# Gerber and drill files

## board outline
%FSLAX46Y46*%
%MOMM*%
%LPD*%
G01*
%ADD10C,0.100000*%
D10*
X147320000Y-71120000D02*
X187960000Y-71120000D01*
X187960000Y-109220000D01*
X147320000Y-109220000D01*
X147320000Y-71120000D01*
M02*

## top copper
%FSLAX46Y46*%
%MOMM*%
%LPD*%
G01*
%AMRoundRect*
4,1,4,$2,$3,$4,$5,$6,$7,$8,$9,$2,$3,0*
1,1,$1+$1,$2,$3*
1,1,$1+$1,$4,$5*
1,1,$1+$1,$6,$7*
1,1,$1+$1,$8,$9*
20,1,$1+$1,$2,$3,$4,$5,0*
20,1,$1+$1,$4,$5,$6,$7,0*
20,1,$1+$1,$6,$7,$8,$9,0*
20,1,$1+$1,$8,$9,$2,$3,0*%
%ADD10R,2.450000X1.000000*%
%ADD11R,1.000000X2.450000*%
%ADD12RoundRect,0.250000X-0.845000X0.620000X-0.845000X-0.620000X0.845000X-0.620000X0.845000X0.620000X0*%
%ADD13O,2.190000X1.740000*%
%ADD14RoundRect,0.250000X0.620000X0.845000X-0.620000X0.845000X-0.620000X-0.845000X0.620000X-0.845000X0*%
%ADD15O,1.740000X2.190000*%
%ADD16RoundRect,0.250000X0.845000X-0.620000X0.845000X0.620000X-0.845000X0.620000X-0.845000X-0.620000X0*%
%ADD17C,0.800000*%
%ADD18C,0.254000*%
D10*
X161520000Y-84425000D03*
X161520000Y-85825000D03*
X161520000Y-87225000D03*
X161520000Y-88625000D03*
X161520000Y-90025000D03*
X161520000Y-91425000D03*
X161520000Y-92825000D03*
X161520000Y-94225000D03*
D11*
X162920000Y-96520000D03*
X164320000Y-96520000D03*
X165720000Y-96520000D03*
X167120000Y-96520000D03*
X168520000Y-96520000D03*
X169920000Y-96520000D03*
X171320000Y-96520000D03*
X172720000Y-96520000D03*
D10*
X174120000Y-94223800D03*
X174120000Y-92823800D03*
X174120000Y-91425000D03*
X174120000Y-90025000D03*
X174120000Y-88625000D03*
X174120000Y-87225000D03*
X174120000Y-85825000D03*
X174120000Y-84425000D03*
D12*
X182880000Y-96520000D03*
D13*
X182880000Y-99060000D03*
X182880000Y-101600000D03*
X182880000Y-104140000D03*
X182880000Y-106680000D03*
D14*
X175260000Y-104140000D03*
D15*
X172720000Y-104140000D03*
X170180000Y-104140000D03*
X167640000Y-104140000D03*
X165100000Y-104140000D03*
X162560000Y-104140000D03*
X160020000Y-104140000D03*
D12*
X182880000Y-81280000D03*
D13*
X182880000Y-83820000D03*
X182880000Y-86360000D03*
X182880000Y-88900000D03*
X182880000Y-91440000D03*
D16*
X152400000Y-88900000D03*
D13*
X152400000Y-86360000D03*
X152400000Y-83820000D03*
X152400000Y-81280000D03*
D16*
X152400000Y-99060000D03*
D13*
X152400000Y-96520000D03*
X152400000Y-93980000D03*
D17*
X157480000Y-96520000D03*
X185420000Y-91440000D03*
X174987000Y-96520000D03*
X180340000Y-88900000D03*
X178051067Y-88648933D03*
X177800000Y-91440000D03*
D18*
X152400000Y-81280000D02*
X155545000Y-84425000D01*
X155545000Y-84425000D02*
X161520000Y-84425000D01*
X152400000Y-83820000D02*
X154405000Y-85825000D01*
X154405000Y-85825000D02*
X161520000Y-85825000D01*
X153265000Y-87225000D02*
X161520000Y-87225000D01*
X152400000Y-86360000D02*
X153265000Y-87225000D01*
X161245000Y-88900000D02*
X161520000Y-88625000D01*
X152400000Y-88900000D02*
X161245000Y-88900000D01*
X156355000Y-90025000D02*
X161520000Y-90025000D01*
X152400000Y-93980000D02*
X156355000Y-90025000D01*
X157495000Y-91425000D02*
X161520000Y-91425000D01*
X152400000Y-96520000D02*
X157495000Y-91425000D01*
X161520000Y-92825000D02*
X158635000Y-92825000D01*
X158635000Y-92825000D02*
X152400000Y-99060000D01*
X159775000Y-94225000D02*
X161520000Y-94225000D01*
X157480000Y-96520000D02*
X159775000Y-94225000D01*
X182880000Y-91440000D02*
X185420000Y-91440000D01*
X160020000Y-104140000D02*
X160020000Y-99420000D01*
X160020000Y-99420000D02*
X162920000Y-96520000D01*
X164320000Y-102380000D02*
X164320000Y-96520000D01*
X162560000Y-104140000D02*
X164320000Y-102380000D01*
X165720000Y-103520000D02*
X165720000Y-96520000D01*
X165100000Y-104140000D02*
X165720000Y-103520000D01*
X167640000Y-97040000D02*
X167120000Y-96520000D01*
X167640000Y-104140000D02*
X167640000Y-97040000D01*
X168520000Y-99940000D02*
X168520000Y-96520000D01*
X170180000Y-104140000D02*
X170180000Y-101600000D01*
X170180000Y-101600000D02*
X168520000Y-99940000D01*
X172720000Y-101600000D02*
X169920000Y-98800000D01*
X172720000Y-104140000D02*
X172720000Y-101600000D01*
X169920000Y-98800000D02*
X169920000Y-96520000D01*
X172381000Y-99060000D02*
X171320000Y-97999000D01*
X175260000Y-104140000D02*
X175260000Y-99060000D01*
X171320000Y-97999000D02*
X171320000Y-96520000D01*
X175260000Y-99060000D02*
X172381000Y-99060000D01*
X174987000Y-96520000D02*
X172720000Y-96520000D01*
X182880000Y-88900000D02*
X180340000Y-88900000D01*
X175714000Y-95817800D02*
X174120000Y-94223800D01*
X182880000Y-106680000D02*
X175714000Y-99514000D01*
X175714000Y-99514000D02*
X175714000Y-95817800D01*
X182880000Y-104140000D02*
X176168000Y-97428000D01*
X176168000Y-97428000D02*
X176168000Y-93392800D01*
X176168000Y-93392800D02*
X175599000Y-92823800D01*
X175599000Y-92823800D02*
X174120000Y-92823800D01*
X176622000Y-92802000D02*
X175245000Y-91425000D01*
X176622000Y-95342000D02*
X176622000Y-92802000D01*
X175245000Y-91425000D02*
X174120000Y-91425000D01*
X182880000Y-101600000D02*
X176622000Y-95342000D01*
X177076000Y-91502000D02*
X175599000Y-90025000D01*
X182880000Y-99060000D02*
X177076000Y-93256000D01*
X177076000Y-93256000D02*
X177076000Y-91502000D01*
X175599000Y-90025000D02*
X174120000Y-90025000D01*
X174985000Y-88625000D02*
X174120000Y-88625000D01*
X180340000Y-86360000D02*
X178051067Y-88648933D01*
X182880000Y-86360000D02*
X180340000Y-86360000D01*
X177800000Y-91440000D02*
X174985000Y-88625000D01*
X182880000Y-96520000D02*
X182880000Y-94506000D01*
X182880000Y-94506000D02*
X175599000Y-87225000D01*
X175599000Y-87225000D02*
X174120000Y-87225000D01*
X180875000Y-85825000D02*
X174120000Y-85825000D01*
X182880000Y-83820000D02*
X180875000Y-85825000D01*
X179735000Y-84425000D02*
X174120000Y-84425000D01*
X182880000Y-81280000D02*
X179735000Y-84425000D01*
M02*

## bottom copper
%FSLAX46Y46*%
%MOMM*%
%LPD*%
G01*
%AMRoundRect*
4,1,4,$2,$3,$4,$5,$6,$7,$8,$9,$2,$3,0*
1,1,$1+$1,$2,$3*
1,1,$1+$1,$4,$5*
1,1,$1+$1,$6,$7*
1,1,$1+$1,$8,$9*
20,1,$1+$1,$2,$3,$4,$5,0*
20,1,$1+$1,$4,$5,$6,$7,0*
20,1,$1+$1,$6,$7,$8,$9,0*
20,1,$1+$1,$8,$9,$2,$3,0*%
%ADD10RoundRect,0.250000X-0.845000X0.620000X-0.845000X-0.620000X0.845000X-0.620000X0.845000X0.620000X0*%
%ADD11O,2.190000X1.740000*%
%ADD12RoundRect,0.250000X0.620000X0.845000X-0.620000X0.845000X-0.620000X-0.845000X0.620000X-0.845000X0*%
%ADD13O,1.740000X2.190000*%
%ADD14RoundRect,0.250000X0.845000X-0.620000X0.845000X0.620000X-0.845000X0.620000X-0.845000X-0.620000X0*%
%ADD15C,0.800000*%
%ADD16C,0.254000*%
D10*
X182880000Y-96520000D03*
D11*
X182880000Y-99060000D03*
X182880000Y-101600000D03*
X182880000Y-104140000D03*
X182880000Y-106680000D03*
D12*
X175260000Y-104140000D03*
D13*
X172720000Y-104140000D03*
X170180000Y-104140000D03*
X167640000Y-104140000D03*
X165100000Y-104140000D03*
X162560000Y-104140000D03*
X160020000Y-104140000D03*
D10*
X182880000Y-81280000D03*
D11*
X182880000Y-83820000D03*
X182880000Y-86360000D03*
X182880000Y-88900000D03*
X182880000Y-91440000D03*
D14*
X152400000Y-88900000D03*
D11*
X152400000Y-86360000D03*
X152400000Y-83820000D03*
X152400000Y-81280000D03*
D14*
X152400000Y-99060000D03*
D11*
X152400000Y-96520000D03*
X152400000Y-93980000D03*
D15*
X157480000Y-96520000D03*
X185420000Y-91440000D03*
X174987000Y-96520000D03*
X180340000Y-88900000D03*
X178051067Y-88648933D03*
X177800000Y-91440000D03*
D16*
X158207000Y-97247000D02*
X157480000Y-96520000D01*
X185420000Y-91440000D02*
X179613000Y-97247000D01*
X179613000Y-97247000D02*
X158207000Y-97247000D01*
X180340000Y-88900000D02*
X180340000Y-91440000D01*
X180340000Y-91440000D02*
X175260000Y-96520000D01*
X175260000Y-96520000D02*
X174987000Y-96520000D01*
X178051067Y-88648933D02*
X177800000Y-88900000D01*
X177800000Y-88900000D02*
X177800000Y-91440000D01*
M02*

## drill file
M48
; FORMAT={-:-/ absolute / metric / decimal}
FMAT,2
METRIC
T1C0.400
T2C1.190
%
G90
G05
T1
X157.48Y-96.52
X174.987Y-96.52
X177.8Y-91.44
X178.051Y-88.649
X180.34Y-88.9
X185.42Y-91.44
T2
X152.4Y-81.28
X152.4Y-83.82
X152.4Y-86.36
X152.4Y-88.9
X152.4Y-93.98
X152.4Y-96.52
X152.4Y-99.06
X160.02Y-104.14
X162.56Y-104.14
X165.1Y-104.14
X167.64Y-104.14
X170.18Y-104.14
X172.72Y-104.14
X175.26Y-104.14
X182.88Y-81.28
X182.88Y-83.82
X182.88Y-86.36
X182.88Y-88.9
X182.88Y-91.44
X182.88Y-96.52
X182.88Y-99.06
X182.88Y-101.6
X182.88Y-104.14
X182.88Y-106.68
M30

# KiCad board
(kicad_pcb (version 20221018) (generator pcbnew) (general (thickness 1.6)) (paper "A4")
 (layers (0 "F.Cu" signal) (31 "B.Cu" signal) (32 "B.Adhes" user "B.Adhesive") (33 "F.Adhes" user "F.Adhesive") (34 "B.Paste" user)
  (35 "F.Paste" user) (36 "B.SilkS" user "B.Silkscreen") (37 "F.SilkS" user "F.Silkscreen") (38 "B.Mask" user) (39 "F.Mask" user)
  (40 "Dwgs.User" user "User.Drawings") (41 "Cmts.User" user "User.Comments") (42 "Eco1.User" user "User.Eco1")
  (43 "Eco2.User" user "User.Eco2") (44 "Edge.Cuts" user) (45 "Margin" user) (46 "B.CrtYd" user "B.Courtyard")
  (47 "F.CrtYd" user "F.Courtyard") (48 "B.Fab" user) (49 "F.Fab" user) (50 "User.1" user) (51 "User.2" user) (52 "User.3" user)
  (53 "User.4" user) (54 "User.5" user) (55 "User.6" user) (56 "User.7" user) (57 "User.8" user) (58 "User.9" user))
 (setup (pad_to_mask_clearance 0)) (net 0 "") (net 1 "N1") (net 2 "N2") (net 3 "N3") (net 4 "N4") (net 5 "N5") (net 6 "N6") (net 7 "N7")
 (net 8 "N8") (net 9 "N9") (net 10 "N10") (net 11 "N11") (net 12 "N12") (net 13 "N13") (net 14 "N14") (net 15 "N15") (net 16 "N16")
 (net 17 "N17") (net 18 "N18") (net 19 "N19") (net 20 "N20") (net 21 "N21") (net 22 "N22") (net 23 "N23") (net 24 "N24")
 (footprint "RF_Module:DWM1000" (layer "F.Cu") (at 167.82 85.2238)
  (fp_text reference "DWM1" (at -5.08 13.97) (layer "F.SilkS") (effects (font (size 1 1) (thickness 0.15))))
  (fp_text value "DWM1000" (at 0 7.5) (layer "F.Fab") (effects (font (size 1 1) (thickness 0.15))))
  (pad "1" smd rect (at -6.3 -0.7988 90) (size 1 2.45) (layers "F.Cu" "F.Paste" "F.Mask") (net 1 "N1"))
  (pad "2" smd rect (at -6.3 0.6012 90) (size 1 2.45) (layers "F.Cu" "F.Paste" "F.Mask") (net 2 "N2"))
  (pad "3" smd rect (at -6.3 2.0012 90) (size 1 2.45) (layers "F.Cu" "F.Paste" "F.Mask") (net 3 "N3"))
  (pad "4" smd rect (at -6.3 3.4012 90) (size 1 2.45) (layers "F.Cu" "F.Paste" "F.Mask") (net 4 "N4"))
  (pad "5" smd rect (at -6.3 4.8012 90) (size 1 2.45) (layers "F.Cu" "F.Paste" "F.Mask") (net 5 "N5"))
  (pad "6" smd rect (at -6.3 6.2012 90) (size 1 2.45) (layers "F.Cu" "F.Paste" "F.Mask") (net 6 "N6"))
  (pad "7" smd rect (at -6.3 7.6012 90) (size 1 2.45) (layers "F.Cu" "F.Paste" "F.Mask") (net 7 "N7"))
  (pad "8" smd rect (at -6.3 9.0012 90) (size 1 2.45) (layers "F.Cu" "F.Paste" "F.Mask") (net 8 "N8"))
  (pad "9" smd rect (at -4.9 11.2962) (size 1 2.45) (layers "F.Cu" "F.Paste" "F.Mask") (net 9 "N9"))
  (pad "10" smd rect (at -3.5 11.2962) (size 1 2.45) (layers "F.Cu" "F.Paste" "F.Mask") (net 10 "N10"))
  (pad "11" smd rect (at -2.1 11.2962) (size 1 2.45) (layers "F.Cu" "F.Paste" "F.Mask") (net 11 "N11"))
  (pad "12" smd rect (at -0.7 11.2962) (size 1 2.45) (layers "F.Cu" "F.Paste" "F.Mask") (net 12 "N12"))
  (pad "13" smd rect (at 0.7 11.2962) (size 1 2.45) (layers "F.Cu" "F.Paste" "F.Mask") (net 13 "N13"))
  (pad "14" smd rect (at 2.1 11.2962) (size 1 2.45) (layers "F.Cu" "F.Paste" "F.Mask") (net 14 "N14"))
  (pad "15" smd rect (at 3.5 11.2962) (size 1 2.45) (layers "F.Cu" "F.Paste" "F.Mask") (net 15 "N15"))
  (pad "16" smd rect (at 4.9 11.2962) (size 1 2.45) (layers "F.Cu" "F.Paste" "F.Mask") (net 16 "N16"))
  (pad "17" smd rect (at 6.3 9 90) (size 1 2.45) (layers "F.Cu" "F.Paste" "F.Mask") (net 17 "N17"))
  (pad "18" smd rect (at 6.3 7.6 90) (size 1 2.45) (layers "F.Cu" "F.Paste" "F.Mask") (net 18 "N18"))
  (pad "19" smd rect (at 6.3 6.2012 90) (size 1 2.45) (layers "F.Cu" "F.Paste" "F.Mask") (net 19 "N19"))
  (pad "20" smd rect (at 6.3 4.8012 90) (size 1 2.45) (layers "F.Cu" "F.Paste" "F.Mask") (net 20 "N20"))
  (pad "21" smd rect (at 6.3 3.4012 90) (size 1 2.45) (layers "F.Cu" "F.Paste" "F.Mask") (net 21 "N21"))
  (pad "22" smd rect (at 6.3 2.0012 90) (size 1 2.45) (layers "F.Cu" "F.Paste" "F.Mask") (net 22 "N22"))
  (pad "23" smd rect (at 6.3 0.6012 90) (size 1 2.45) (layers "F.Cu" "F.Paste" "F.Mask") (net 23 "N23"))
  (pad "24" smd rect (at 6.3 -0.7988 90) (size 1 2.45) (layers "F.Cu" "F.Paste" "F.Mask") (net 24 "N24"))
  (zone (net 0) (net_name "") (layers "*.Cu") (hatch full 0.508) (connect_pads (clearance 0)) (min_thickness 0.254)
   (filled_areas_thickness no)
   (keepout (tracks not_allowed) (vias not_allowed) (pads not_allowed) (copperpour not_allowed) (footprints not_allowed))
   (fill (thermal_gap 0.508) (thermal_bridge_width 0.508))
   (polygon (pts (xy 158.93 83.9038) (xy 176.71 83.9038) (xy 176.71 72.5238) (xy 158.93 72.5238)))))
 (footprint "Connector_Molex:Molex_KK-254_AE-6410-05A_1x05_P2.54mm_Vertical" (layer "F.Cu") (at 182.88 96.52 -90)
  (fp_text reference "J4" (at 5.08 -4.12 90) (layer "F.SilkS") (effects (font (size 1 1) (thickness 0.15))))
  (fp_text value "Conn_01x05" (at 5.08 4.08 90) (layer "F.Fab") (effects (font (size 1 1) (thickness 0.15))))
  (pad "1" thru_hole roundrect (at 0 0 270) (size 1.74 2.19) (drill 1.19) (layers "*.Cu" "*.Mask") (roundrect_rratio 0.1436781609)
   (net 22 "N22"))
  (pad "2" thru_hole oval (at 2.54 0 270) (size 1.74 2.19) (drill 1.19) (layers "*.Cu" "*.Mask") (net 20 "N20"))
  (pad "3" thru_hole oval (at 5.08 0 270) (size 1.74 2.19) (drill 1.19) (layers "*.Cu" "*.Mask") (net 19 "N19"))
  (pad "4" thru_hole oval (at 7.62 0 270) (size 1.74 2.19) (drill 1.19) (layers "*.Cu" "*.Mask") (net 18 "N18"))
  (pad "5" thru_hole oval (at 10.16 0 270) (size 1.74 2.19) (drill 1.19) (layers "*.Cu" "*.Mask") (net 17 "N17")))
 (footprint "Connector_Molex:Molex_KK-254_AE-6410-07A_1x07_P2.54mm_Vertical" (layer "F.Cu") (at 175.26 104.14 180)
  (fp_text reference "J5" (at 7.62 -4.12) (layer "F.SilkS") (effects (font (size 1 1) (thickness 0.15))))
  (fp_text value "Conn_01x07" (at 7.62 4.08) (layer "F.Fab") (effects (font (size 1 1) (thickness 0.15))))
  (pad "1" thru_hole roundrect (at 0 0 180) (size 1.74 2.19) (drill 1.19) (layers "*.Cu" "*.Mask") (roundrect_rratio 0.1436781609)
   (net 15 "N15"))
  (pad "2" thru_hole oval (at 2.54 0 180) (size 1.74 2.19) (drill 1.19) (layers "*.Cu" "*.Mask") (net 14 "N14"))
  (pad "3" thru_hole oval (at 5.08 0 180) (size 1.74 2.19) (drill 1.19) (layers "*.Cu" "*.Mask") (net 13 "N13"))
  (pad "4" thru_hole oval (at 7.62 0 180) (size 1.74 2.19) (drill 1.19) (layers "*.Cu" "*.Mask") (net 12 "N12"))
  (pad "5" thru_hole oval (at 10.16 0 180) (size 1.74 2.19) (drill 1.19) (layers "*.Cu" "*.Mask") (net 11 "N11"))
  (pad "6" thru_hole oval (at 12.7 0 180) (size 1.74 2.19) (drill 1.19) (layers "*.Cu" "*.Mask") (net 10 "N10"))
  (pad "7" thru_hole oval (at 15.24 0 180) (size 1.74 2.19) (drill 1.19) (layers "*.Cu" "*.Mask") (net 9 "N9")))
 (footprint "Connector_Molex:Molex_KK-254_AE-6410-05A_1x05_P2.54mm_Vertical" (layer "F.Cu") (at 182.88 81.28 -90)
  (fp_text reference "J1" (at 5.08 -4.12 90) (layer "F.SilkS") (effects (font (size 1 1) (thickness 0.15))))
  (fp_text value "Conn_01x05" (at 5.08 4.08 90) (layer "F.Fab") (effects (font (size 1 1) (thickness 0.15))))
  (pad "1" thru_hole roundrect (at 0 0 270) (size 1.74 2.19) (drill 1.19) (layers "*.Cu" "*.Mask") (roundrect_rratio 0.1436781609)
   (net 24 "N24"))
  (pad "2" thru_hole oval (at 2.54 0 270) (size 1.74 2.19) (drill 1.19) (layers "*.Cu" "*.Mask") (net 23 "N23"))
  (pad "3" thru_hole oval (at 5.08 0 270) (size 1.74 2.19) (drill 1.19) (layers "*.Cu" "*.Mask") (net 21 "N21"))
  (pad "4" thru_hole oval (at 7.62 0 270) (size 1.74 2.19) (drill 1.19) (layers "*.Cu" "*.Mask") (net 16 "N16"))
  (pad "5" thru_hole oval (at 10.16 0 270) (size 1.74 2.19) (drill 1.19) (layers "*.Cu" "*.Mask") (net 8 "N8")))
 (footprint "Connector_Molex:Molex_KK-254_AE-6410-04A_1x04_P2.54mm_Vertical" (layer "F.Cu") (at 152.4 88.9 90)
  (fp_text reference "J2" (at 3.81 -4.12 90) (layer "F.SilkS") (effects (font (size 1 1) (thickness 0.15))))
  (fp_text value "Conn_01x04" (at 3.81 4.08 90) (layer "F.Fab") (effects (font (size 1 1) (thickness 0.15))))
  (pad "1" thru_hole roundrect (at 0 0 90) (size 1.74 2.19) (drill 1.19) (layers "*.Cu" "*.Mask") (roundrect_rratio 0.1436781609)
   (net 4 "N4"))
  (pad "2" thru_hole oval (at 2.54 0 90) (size 1.74 2.19) (drill 1.19) (layers "*.Cu" "*.Mask") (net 3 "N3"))
  (pad "3" thru_hole oval (at 5.08 0 90) (size 1.74 2.19) (drill 1.19) (layers "*.Cu" "*.Mask") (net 2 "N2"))
  (pad "4" thru_hole oval (at 7.62 0 90) (size 1.74 2.19) (drill 1.19) (layers "*.Cu" "*.Mask") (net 1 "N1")))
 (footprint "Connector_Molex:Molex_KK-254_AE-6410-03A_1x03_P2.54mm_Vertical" (layer "F.Cu") (at 152.4 99.06 90)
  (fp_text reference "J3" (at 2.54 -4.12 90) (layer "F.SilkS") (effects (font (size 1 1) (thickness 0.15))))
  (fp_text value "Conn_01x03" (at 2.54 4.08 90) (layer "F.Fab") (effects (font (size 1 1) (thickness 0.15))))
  (pad "1" thru_hole roundrect (at 0 0 90) (size 1.74 2.19) (drill 1.19) (layers "*.Cu" "*.Mask") (roundrect_rratio 0.1436781609)
   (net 7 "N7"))
  (pad "2" thru_hole oval (at 2.54 0 90) (size 1.74 2.19) (drill 1.19) (layers "*.Cu" "*.Mask") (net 6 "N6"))
  (pad "3" thru_hole oval (at 5.08 0 90) (size 1.74 2.19) (drill 1.19) (layers "*.Cu" "*.Mask") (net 5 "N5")))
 (gr_rect (start 147.32 71.12) (end 187.96 109.22) (stroke (width 0.1) (type default)) (fill none) (layer "Edge.Cuts"))
 (segment (start 152.4 81.28) (end 155.545 84.425) (width 0.254) (layer "F.Cu") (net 1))
 (segment (start 155.545 84.425) (end 161.52 84.425) (width 0.254) (layer "F.Cu") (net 1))
 (segment (start 152.4 83.82) (end 154.405 85.825) (width 0.254) (layer "F.Cu") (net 2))
 (segment (start 154.405 85.825) (end 161.52 85.825) (width 0.254) (layer "F.Cu") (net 2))
 (segment (start 153.265 87.225) (end 161.52 87.225) (width 0.254) (layer "F.Cu") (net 3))
 (segment (start 152.4 86.36) (end 153.265 87.225) (width 0.254) (layer "F.Cu") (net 3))
 (segment (start 161.245 88.9) (end 161.52 88.625) (width 0.254) (layer "F.Cu") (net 4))
 (segment (start 152.4 88.9) (end 161.245 88.9) (width 0.254) (layer "F.Cu") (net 4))
 (segment (start 156.355 90.025) (end 161.52 90.025) (width 0.254) (layer "F.Cu") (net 5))
 (segment (start 152.4 93.98) (end 156.355 90.025) (width 0.254) (layer "F.Cu") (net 5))
 (segment (start 157.495 91.425) (end 161.52 91.425) (width 0.254) (layer "F.Cu") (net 6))
 (segment (start 152.4 96.52) (end 157.495 91.425) (width 0.254) (layer "F.Cu") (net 6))
 (segment (start 161.52 92.825) (end 158.635 92.825) (width 0.254) (layer "F.Cu") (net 7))
 (segment (start 158.635 92.825) (end 152.4 99.06) (width 0.254) (layer "F.Cu") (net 7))
 (segment (start 159.775 94.225) (end 161.52 94.225) (width 0.254) (layer "F.Cu") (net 8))
 (segment (start 157.48 96.52) (end 159.775 94.225) (width 0.254) (layer "F.Cu") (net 8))
 (segment (start 182.88 91.44) (end 185.42 91.44) (width 0.254) (layer "F.Cu") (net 8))
 (via (at 157.48 96.52) (size 0.8) (drill 0.4) (layers "F.Cu" "B.Cu") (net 8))
 (via (at 185.42 91.44) (size 0.8) (drill 0.4) (layers "F.Cu" "B.Cu") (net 8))
 (segment (start 158.207 97.247) (end 157.48 96.52) (width 0.254) (layer "B.Cu") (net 8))
 (segment (start 185.42 91.44) (end 179.613 97.247) (width 0.254) (layer "B.Cu") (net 8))
 (segment (start 179.613 97.247) (end 158.207 97.247) (width 0.254) (layer "B.Cu") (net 8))
 (segment (start 160.02 104.14) (end 160.02 99.42) (width 0.254) (layer "F.Cu") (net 9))
 (segment (start 160.02 99.42) (end 162.92 96.52) (width 0.254) (layer "F.Cu") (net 9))
 (segment (start 164.32 102.38) (end 164.32 96.52) (width 0.254) (layer "F.Cu") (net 10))
 (segment (start 162.56 104.14) (end 164.32 102.38) (width 0.254) (layer "F.Cu") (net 10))
 (segment (start 165.72 103.52) (end 165.72 96.52) (width 0.254) (layer "F.Cu") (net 11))
 (segment (start 165.1 104.14) (end 165.72 103.52) (width 0.254) (layer "F.Cu") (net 11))
 (segment (start 167.64 97.04) (end 167.12 96.52) (width 0.254) (layer "F.Cu") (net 12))
 (segment (start 167.64 104.14) (end 167.64 97.04) (width 0.254) (layer "F.Cu") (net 12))
 (segment (start 168.52 99.94) (end 168.52 96.52) (width 0.254) (layer "F.Cu") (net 13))
 (segment (start 170.18 104.14) (end 170.18 101.6) (width 0.254) (layer "F.Cu") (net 13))
 (segment (start 170.18 101.6) (end 168.52 99.94) (width 0.254) (layer "F.Cu") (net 13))
 (segment (start 172.72 101.6) (end 169.92 98.8) (width 0.254) (layer "F.Cu") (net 14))
 (segment (start 172.72 104.14) (end 172.72 101.6) (width 0.254) (layer "F.Cu") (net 14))
 (segment (start 169.92 98.8) (end 169.92 96.52) (width 0.254) (layer "F.Cu") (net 14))
 (segment (start 172.381 99.06) (end 171.32 97.999) (width 0.254) (layer "F.Cu") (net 15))
 (segment (start 175.26 104.14) (end 175.26 99.06) (width 0.254) (layer "F.Cu") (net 15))
 (segment (start 171.32 97.999) (end 171.32 96.52) (width 0.254) (layer "F.Cu") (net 15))
 (segment (start 175.26 99.06) (end 172.381 99.06) (width 0.254) (layer "F.Cu") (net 15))
 (segment (start 174.987 96.52) (end 172.72 96.52) (width 0.254) (layer "F.Cu") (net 16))
 (segment (start 182.88 88.9) (end 180.34 88.9) (width 0.254) (layer "F.Cu") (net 16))
 (via (at 174.987 96.52) (size 0.8) (drill 0.4) (layers "F.Cu" "B.Cu") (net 16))
 (via (at 180.34 88.9) (size 0.8) (drill 0.4) (layers "F.Cu" "B.Cu") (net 16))
 (segment (start 180.34 88.9) (end 180.34 91.44) (width 0.254) (layer "B.Cu") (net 16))
 (segment (start 180.34 91.44) (end 175.26 96.52) (width 0.254) (layer "B.Cu") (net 16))
 (segment (start 175.26 96.52) (end 174.987 96.52) (width 0.254) (layer "B.Cu") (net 16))
 (segment (start 175.714 95.8178) (end 174.12 94.2238) (width 0.254) (layer "F.Cu") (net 17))
 (segment (start 182.88 106.68) (end 175.714 99.514) (width 0.254) (layer "F.Cu") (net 17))
 (segment (start 175.714 99.514) (end 175.714 95.8178) (width 0.254) (layer "F.Cu") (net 17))
 (segment (start 182.88 104.14) (end 176.168 97.428) (width 0.254) (layer "F.Cu") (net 18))
 (segment (start 176.168 97.428) (end 176.168 93.3928) (width 0.254) (layer "F.Cu") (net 18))
 (segment (start 176.168 93.3928) (end 175.599 92.8238) (width 0.254) (layer "F.Cu") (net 18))
 (segment (start 175.599 92.8238) (end 174.12 92.8238) (width 0.254) (layer "F.Cu") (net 18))
 (segment (start 176.622 92.802) (end 175.245 91.425) (width 0.254) (layer "F.Cu") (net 19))
 (segment (start 176.622 95.342) (end 176.622 92.802) (width 0.254) (layer "F.Cu") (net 19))
 (segment (start 175.245 91.425) (end 174.12 91.425) (width 0.254) (layer "F.Cu") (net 19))
 (segment (start 182.88 101.6) (end 176.622 95.342) (width 0.254) (layer "F.Cu") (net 19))
 (segment (start 177.076 91.502) (end 175.599 90.025) (width 0.254) (layer "F.Cu") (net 20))
 (segment (start 182.88 99.06) (end 177.076 93.256) (width 0.254) (layer "F.Cu") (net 20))
 (segment (start 177.076 93.256) (end 177.076 91.502) (width 0.254) (layer "F.Cu") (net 20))
 (segment (start 175.599 90.025) (end 174.12 90.025) (width 0.254) (layer "F.Cu") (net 20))
 (segment (start 174.985 88.625) (end 174.12 88.625) (width 0.254) (layer "F.Cu") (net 21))
 (segment (start 180.34 86.36) (end 178.051067 88.648933) (width 0.254) (layer "F.Cu") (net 21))
 (segment (start 182.88 86.36) (end 180.34 86.36) (width 0.254) (layer "F.Cu") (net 21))
 (segment (start 177.8 91.44) (end 174.985 88.625) (width 0.254) (layer "F.Cu") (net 21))
 (via (at 178.051067 88.648933) (size 0.8) (drill 0.4) (layers "F.Cu" "B.Cu") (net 21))
 (via (at 177.8 91.44) (size 0.8) (drill 0.4) (layers "F.Cu" "B.Cu") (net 21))
 (segment (start 178.051067 88.648933) (end 177.8 88.9) (width 0.254) (layer "B.Cu") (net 21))
 (segment (start 177.8 88.9) (end 177.8 91.44) (width 0.254) (layer "B.Cu") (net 21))
 (segment (start 182.88 96.52) (end 182.88 94.506) (width 0.254) (layer "F.Cu") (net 22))
 (segment (start 182.88 94.506) (end 175.599 87.225) (width 0.254) (layer "F.Cu") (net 22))
 (segment (start 175.599 87.225) (end 174.12 87.225) (width 0.254) (layer "F.Cu") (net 22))
 (segment (start 180.875 85.825) (end 174.12 85.825) (width 0.254) (layer "F.Cu") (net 23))
 (segment (start 182.88 83.82) (end 180.875 85.825) (width 0.254) (layer "F.Cu") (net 23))
 (segment (start 179.735 84.425) (end 174.12 84.425) (width 0.254) (layer "F.Cu") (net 24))
 (segment (start 182.88 81.28) (end 179.735 84.425) (width 0.254) (layer "F.Cu") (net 24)))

